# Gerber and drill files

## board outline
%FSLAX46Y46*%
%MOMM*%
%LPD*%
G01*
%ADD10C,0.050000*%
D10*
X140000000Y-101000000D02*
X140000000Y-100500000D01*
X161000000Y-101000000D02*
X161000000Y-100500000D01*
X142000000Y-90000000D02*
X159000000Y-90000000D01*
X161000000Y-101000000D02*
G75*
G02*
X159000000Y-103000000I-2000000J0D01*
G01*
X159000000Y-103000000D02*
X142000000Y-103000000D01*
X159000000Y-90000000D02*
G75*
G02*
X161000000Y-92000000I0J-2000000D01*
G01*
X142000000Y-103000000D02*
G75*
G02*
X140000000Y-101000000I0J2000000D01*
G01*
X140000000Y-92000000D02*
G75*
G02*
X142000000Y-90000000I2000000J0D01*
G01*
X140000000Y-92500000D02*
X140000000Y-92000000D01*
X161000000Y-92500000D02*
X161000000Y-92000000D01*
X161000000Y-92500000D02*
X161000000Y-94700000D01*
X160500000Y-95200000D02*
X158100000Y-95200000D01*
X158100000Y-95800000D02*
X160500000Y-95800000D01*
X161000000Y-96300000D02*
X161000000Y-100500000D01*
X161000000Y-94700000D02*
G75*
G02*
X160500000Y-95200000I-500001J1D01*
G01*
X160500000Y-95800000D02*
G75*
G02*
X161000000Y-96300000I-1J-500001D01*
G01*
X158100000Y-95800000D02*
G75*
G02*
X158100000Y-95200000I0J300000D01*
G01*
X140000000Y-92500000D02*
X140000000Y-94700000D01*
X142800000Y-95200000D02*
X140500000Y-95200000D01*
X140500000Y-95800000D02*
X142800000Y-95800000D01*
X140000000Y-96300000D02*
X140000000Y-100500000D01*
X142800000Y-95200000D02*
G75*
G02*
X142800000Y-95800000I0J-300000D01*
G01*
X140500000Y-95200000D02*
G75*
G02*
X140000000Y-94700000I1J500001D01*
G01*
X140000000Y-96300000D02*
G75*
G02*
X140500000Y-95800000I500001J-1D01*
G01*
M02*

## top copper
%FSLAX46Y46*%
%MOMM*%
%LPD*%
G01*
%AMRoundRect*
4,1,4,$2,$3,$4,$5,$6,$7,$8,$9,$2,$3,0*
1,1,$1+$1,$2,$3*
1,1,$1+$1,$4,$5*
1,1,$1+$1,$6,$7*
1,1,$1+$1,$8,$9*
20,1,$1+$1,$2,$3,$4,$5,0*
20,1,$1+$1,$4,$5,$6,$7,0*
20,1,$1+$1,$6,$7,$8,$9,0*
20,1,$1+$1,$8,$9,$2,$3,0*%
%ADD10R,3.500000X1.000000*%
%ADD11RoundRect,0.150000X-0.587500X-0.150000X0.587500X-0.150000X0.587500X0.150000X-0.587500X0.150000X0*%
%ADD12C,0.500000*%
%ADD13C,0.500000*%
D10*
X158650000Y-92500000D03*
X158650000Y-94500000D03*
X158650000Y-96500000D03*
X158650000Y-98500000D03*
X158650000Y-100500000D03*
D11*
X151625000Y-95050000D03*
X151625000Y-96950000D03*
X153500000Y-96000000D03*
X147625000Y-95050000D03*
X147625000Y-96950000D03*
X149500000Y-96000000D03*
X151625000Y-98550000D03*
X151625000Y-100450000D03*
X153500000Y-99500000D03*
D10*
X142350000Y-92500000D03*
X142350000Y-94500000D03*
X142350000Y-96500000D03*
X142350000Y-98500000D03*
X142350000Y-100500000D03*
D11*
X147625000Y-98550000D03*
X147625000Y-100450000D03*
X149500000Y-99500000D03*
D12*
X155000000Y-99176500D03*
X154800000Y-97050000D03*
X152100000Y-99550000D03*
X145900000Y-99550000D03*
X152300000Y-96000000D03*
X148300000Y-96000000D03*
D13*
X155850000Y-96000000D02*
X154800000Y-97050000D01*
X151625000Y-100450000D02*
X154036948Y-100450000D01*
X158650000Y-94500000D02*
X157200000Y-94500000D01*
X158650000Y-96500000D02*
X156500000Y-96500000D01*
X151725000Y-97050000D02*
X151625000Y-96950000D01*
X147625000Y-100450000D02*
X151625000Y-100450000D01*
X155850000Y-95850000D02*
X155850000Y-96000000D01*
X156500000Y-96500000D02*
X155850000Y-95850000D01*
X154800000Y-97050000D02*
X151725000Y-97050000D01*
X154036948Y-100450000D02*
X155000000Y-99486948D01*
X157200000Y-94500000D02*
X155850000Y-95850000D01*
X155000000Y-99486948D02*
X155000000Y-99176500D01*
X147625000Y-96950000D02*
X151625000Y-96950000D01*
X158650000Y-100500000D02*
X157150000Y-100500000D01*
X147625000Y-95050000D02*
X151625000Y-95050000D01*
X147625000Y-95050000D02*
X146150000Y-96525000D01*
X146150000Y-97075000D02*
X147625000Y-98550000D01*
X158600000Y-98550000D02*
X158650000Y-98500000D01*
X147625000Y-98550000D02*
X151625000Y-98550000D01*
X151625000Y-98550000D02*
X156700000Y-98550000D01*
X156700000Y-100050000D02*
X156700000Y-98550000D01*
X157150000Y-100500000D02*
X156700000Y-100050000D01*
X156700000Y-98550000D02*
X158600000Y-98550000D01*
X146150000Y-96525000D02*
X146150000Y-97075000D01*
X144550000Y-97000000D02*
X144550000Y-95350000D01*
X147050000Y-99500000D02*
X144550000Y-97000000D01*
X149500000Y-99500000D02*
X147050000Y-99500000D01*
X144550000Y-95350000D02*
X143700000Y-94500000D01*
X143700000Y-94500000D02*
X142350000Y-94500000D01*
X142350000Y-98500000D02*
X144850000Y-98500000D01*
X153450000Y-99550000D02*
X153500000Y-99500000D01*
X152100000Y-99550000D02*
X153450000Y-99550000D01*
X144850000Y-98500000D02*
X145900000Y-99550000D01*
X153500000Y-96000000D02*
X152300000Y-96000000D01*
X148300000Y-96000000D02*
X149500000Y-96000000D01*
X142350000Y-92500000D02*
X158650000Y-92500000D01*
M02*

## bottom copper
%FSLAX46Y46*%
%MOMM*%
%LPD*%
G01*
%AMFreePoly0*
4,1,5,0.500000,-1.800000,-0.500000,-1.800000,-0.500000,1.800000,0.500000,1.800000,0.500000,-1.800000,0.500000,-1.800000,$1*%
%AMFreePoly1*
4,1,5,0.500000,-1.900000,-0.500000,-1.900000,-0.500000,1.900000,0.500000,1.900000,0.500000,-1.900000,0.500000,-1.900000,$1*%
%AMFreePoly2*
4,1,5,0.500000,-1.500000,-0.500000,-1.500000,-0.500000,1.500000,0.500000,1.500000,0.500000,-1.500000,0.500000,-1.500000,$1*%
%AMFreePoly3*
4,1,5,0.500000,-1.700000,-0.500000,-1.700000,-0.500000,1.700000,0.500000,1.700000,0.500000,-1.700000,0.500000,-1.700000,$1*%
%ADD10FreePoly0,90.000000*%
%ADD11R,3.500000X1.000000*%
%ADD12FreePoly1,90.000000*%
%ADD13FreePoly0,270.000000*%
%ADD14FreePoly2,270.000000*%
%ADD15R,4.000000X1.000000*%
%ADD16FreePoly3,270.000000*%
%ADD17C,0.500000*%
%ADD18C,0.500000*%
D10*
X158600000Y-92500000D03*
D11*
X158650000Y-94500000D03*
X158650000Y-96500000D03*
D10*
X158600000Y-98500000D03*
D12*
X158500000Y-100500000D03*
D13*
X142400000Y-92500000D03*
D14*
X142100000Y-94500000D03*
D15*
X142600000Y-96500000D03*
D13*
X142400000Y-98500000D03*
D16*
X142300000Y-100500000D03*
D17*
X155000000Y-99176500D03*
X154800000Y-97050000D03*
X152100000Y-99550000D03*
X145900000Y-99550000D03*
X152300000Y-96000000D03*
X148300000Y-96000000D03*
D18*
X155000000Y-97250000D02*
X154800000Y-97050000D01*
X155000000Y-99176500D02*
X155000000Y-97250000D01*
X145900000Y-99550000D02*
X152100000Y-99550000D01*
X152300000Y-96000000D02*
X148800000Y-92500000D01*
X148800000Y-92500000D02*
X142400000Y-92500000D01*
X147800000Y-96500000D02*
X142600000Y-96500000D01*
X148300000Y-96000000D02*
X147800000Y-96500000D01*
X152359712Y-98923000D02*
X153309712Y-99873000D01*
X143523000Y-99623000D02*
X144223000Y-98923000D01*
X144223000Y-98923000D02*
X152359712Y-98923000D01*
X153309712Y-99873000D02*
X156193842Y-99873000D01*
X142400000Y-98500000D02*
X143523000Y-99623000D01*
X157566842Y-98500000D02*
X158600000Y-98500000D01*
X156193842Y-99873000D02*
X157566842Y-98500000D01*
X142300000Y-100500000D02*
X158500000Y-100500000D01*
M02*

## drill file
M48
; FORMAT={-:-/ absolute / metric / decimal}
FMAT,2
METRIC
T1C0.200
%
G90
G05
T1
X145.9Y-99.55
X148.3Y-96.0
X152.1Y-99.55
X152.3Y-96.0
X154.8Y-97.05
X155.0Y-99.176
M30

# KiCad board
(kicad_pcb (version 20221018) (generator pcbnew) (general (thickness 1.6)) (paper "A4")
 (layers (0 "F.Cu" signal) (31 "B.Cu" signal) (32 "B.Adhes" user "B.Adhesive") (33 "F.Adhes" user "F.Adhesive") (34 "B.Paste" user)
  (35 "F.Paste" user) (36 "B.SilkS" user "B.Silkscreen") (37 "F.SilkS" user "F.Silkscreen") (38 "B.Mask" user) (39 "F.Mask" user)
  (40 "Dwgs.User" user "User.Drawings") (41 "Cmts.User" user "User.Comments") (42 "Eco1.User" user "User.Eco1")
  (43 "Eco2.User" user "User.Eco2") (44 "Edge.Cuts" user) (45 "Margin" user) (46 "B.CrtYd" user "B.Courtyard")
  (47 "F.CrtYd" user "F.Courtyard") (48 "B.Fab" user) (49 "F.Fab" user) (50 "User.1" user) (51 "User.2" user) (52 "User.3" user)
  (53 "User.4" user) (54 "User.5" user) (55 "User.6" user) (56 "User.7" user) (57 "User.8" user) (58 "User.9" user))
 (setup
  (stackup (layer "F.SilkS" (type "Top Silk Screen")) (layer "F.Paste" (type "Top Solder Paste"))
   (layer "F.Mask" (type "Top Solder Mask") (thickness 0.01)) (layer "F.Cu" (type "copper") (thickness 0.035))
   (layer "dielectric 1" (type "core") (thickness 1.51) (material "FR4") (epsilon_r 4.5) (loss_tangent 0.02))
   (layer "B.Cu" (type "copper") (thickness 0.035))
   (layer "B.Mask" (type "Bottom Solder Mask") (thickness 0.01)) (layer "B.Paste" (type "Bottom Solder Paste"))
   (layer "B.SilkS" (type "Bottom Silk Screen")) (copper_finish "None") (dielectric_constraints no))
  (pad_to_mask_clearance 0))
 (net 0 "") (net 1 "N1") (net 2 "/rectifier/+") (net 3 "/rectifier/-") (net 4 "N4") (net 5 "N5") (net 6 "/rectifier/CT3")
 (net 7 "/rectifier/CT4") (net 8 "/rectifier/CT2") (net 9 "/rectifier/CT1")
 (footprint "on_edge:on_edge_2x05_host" (layer "F.Cu") (at 161 96.5 -90)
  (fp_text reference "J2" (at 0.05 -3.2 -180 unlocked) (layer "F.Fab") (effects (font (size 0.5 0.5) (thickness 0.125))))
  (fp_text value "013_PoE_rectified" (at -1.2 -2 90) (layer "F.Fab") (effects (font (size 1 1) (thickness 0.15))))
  (fp_line (start -4 0) (end -1.8 0) (stroke (width 0.05) (type solid)) (layer "Edge.Cuts"))
  (fp_line (start -1.3 0.5) (end -1.3 2.9) (stroke (width 0.05) (type solid)) (layer "Edge.Cuts"))
  (fp_line (start -0.7 2.9) (end -0.7 0.5) (stroke (width 0.05) (type solid)) (layer "Edge.Cuts"))
  (fp_line (start -0.2 0) (end 4 0) (stroke (width 0.05) (type solid)) (layer "Edge.Cuts"))
  (fp_arc (start -1.8 0) (mid -1.446447 0.146447) (end -1.3 0.5) (stroke (width 0.05) (type solid)) (layer "Edge.Cuts"))
  (fp_arc (start -0.7 0.5) (mid -0.553553 0.146447) (end -0.2 0) (stroke (width 0.05) (type solid)) (layer "Edge.Cuts"))
  (fp_arc (start -0.7 2.9) (mid -1 3.2) (end -1.3 2.9) (stroke (width 0.05) (type solid)) (layer "Edge.Cuts"))
  (pad "1" smd rect (at -4 2.35 270) (size 1 3.5) (layers "F.Cu" "F.Mask") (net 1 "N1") (zone_connect 0))
  (pad "2" smd rect (at -2 2.35 270) (size 1 3.5) (layers "F.Cu" "F.Mask") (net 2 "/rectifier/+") (zone_connect 0))
  (pad "3" smd rect (at 0 2.35 270) (size 1 3.5) (layers "F.Cu" "F.Mask") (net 2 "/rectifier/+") (zone_connect 0))
  (pad "4" smd rect (at 2 2.35 270) (size 1 3.5) (layers "F.Cu" "F.Mask") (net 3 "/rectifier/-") (zone_connect 0))
  (pad "5" smd rect (at 4 2.35 270) (size 1 3.5) (layers "F.Cu" "F.Mask") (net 3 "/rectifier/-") (zone_connect 0))
  (pad "6" smd custom (at -4 2.4 90) (size 1 3.6) (layers "B.Cu" "B.Mask") (zone_connect 0) (options (clearance outline) (anchor rect))
   (primitives))
  (pad "7" smd rect (at -2 2.35 90) (size 1 3.5) (layers "B.Cu" "B.Mask") (zone_connect 0))
  (pad "8" smd rect (at 0 2.35 90) (size 1 3.5) (layers "B.Cu" "B.Mask") (zone_connect 0))
  (pad "9" smd custom (at 2 2.4 90) (size 1 3.6) (layers "B.Cu" "B.Mask") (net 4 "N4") (zone_connect 0)
   (options (clearance outline) (anchor rect)) (primitives))
  (pad "10" smd custom (at 4 2.5 90) (size 1 3.8) (layers "B.Cu" "B.Mask") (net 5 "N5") (zone_connect 0)
   (options (clearance outline) (anchor rect)) (primitives))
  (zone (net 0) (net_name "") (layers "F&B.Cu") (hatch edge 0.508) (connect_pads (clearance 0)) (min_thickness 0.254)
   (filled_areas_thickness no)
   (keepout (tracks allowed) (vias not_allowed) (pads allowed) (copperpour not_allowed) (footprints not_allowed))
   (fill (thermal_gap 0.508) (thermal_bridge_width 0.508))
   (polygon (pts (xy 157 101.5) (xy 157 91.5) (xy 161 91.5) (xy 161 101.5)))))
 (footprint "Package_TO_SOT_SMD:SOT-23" (layer "F.Cu") (at 152.5625 96)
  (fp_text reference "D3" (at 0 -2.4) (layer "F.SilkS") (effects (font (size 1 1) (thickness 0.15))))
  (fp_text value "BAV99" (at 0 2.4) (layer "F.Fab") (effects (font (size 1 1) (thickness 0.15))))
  (pad "1" smd roundrect (at -0.9375 -0.95) (size 1.475 0.6) (layers "F.Cu" "F.Paste" "F.Mask") (roundrect_rratio 0.25)
   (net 3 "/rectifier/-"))
  (pad "2" smd roundrect (at -0.9375 0.95) (size 1.475 0.6) (layers "F.Cu" "F.Paste" "F.Mask") (roundrect_rratio 0.25)
   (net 2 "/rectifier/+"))
  (pad "3" smd roundrect (at 0.9375 0) (size 1.475 0.6) (layers "F.Cu" "F.Paste" "F.Mask") (roundrect_rratio 0.25) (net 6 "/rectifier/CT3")))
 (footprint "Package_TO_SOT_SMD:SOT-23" (layer "F.Cu") (at 148.5625 96)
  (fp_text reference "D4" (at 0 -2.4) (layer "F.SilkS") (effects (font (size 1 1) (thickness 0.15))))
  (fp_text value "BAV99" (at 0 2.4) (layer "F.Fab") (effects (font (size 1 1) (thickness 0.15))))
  (pad "1" smd roundrect (at -0.9375 -0.95) (size 1.475 0.6) (layers "F.Cu" "F.Paste" "F.Mask") (roundrect_rratio 0.25)
   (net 3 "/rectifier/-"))
  (pad "2" smd roundrect (at -0.9375 0.95) (size 1.475 0.6) (layers "F.Cu" "F.Paste" "F.Mask") (roundrect_rratio 0.25)
   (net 2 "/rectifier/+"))
  (pad "3" smd roundrect (at 0.9375 0) (size 1.475 0.6) (layers "F.Cu" "F.Paste" "F.Mask") (roundrect_rratio 0.25) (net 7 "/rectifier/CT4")))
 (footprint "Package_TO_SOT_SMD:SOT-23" (layer "F.Cu") (at 152.5625 99.5)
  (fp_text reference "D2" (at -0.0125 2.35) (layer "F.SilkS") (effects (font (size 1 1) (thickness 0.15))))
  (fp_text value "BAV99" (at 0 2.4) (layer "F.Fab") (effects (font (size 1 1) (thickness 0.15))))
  (pad "1" smd roundrect (at -0.9375 -0.95) (size 1.475 0.6) (layers "F.Cu" "F.Paste" "F.Mask") (roundrect_rratio 0.25)
   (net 3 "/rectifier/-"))
  (pad "2" smd roundrect (at -0.9375 0.95) (size 1.475 0.6) (layers "F.Cu" "F.Paste" "F.Mask") (roundrect_rratio 0.25)
   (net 2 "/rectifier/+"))
  (pad "3" smd roundrect (at 0.9375 0) (size 1.475 0.6) (layers "F.Cu" "F.Paste" "F.Mask") (roundrect_rratio 0.25) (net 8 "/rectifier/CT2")))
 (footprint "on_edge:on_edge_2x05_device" (layer "F.Cu") (at 140 96.5 -90)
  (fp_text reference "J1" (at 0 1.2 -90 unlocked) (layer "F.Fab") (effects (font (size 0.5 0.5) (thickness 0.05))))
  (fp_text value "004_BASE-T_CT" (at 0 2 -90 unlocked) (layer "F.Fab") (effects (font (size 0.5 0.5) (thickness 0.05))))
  (fp_line (start -4 0) (end -1.8 0) (stroke (width 0.05) (type solid)) (layer "Edge.Cuts"))
  (fp_line (start -1.3 -2.8) (end -1.3 -0.5) (stroke (width 0.05) (type solid)) (layer "Edge.Cuts"))
  (fp_line (start -0.7 -0.5) (end -0.7 -2.8) (stroke (width 0.05) (type solid)) (layer "Edge.Cuts"))
  (fp_line (start -0.2 0) (end 4 0) (stroke (width 0.05) (type solid)) (layer "Edge.Cuts"))
  (fp_arc (start -1.3 -2.8) (mid -1 -3.1) (end -0.7 -2.8) (stroke (width 0.05) (type solid)) (layer "Edge.Cuts"))
  (fp_arc (start -1.3 -0.5) (mid -1.446447 -0.146447) (end -1.8 0) (stroke (width 0.05) (type solid)) (layer "Edge.Cuts"))
  (fp_arc (start -0.2 0) (mid -0.553553 -0.146447) (end -0.7 -0.5) (stroke (width 0.05) (type solid)) (layer "Edge.Cuts"))
  (pad "1" smd rect (at -4 -2.35 90) (size 1 3.5) (layers "F.Cu" "F.Mask") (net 1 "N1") (zone_connect 0))
  (pad "2" smd rect (at -2 -2.35 270) (size 1 3.5) (layers "F.Cu" "F.Mask") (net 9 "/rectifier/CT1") (zone_connect 0))
  (pad "3" smd rect (at 0 -2.35 270) (size 1 3.5) (layers "F.Cu" "F.Mask") (zone_connect 0))
  (pad "4" smd rect (at 2 -2.35 90) (size 1 3.5) (layers "F.Cu" "F.Mask") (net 8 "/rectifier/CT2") (zone_connect 0))
  (pad "5" smd rect (at 4 -2.35 90) (size 1 3.5) (layers "F.Cu" "F.Mask") (zone_connect 0))
  (pad "6" smd custom (at -4 -2.4 270) (size 1 3.6) (layers "B.Cu" "B.Mask") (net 6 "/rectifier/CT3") (zone_connect 0)
   (options (clearance outline) (anchor rect)) (primitives))
  (pad "7" smd custom (at -2 -2.1 270) (size 1 3) (layers "B.Cu" "B.Mask") (zone_connect 0) (options (clearance outline) (anchor rect))
   (primitives))
  (pad "8" smd rect (at 0 -2.6 270) (size 1 4) (layers "B.Cu" "B.Mask") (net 7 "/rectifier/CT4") (zone_connect 0))
  (pad "9" smd custom (at 2 -2.4 270) (size 1 3.6) (layers "B.Cu" "B.Mask") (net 4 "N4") (zone_connect 0)
   (options (clearance outline) (anchor rect)) (primitives))
  (pad "10" smd custom (at 4 -2.3 270) (size 1 3.4) (layers "B.Cu" "B.Mask") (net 5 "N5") (zone_connect 0)
   (options (clearance outline) (anchor rect)) (primitives))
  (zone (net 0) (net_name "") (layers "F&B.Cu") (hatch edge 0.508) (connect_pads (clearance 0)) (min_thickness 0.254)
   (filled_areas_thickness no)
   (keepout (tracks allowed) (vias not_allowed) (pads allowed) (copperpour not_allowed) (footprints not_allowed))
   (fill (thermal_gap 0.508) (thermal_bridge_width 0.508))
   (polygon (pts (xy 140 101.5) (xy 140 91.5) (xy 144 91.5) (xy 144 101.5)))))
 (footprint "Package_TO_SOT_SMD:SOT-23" (layer "F.Cu") (at 148.5625 99.5)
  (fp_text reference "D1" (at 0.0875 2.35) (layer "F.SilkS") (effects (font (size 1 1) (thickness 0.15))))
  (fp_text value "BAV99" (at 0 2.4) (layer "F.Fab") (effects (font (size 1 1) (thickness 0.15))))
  (pad "1" smd roundrect (at -0.9375 -0.95) (size 1.475 0.6) (layers "F.Cu" "F.Paste" "F.Mask") (roundrect_rratio 0.25)
   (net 3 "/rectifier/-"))
  (pad "2" smd roundrect (at -0.9375 0.95) (size 1.475 0.6) (layers "F.Cu" "F.Paste" "F.Mask") (roundrect_rratio 0.25)
   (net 2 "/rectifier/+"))
  (pad "3" smd roundrect (at 0.9375 0) (size 1.475 0.6) (layers "F.Cu" "F.Paste" "F.Mask") (roundrect_rratio 0.25) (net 9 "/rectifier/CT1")))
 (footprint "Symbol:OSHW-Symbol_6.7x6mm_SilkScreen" (layer "B.Cu") (at 152.45 99.75 180)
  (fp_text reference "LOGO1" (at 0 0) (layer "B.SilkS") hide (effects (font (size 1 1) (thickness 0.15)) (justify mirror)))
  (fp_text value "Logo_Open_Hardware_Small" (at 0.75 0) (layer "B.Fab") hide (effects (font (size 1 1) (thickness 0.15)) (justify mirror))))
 (gr_line (start 140 101) (end 140 100.5) (stroke (width 0.05) (type solid)) (layer "Edge.Cuts"))
 (gr_line (start 161 101) (end 161 100.5) (stroke (width 0.05) (type solid)) (layer "Edge.Cuts"))
 (gr_line (start 142 90) (end 159 90) (stroke (width 0.05) (type solid)) (layer "Edge.Cuts"))
 (gr_arc (start 161 101) (mid 160.414214 102.414214) (end 159 103) (stroke (width 0.05) (type solid)) (layer "Edge.Cuts"))
 (gr_line (start 159 103) (end 142 103) (stroke (width 0.05) (type solid)) (layer "Edge.Cuts"))
 (gr_arc (start 159 90) (mid 160.414214 90.585786) (end 161 92) (stroke (width 0.05) (type solid)) (layer "Edge.Cuts"))
 (gr_arc (start 142 103) (mid 140.585786 102.414214) (end 140 101) (stroke (width 0.05) (type solid)) (layer "Edge.Cuts"))
 (gr_arc (start 140 92) (mid 140.585786 90.585786) (end 142 90) (stroke (width 0.05) (type solid)) (layer "Edge.Cuts"))
 (gr_line (start 140 92.5) (end 140 92) (stroke (width 0.05) (type solid)) (layer "Edge.Cuts"))
 (gr_line (start 161 92.5) (end 161 92) (stroke (width 0.05) (type solid)) (layer "Edge.Cuts"))
 (segment (start 155.85 96) (end 154.8 97.05) (width 0.5) (layer "F.Cu") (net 2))
 (segment (start 151.625 100.45) (end 154.036948 100.45) (width 0.5) (layer "F.Cu") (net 2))
 (segment (start 158.65 94.5) (end 157.2 94.5) (width 0.5) (layer "F.Cu") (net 2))
 (segment (start 158.65 96.5) (end 156.5 96.5) (width 0.5) (layer "F.Cu") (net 2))
 (segment (start 151.725 97.05) (end 151.625 96.95) (width 0.5) (layer "F.Cu") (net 2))
 (segment (start 147.625 100.45) (end 151.625 100.45) (width 0.5) (layer "F.Cu") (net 2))
 (segment (start 155.85 95.85) (end 155.85 96) (width 0.5) (layer "F.Cu") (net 2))
 (segment (start 156.5 96.5) (end 155.85 95.85) (width 0.5) (layer "F.Cu") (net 2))
 (segment (start 154.8 97.05) (end 151.725 97.05) (width 0.5) (layer "F.Cu") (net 2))
 (segment (start 154.036948 100.45) (end 155 99.486948) (width 0.5) (layer "F.Cu") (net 2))
 (segment (start 157.2 94.5) (end 155.85 95.85) (width 0.5) (layer "F.Cu") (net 2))
 (segment (start 155 99.486948) (end 155 99.1765) (width 0.5) (layer "F.Cu") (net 2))
 (segment (start 147.625 96.95) (end 151.625 96.95) (width 0.5) (layer "F.Cu") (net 2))
 (via (at 155 99.1765) (size 0.5) (drill 0.2) (layers "F.Cu" "B.Cu") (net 2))
 (via (at 154.8 97.05) (size 0.5) (drill 0.2) (layers "F.Cu" "B.Cu") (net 2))
 (segment (start 155 97.25) (end 154.8 97.05) (width 0.5) (layer "B.Cu") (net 2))
 (segment (start 155 99.1765) (end 155 97.25) (width 0.5) (layer "B.Cu") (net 2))
 (segment (start 158.65 100.5) (end 157.15 100.5) (width 0.5) (layer "F.Cu") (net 3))
 (segment (start 147.625 95.05) (end 151.625 95.05) (width 0.5) (layer "F.Cu") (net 3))
 (segment (start 147.625 95.05) (end 146.15 96.525) (width 0.5) (layer "F.Cu") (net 3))
 (segment (start 146.15 97.075) (end 147.625 98.55) (width 0.5) (layer "F.Cu") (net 3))
 (segment (start 158.6 98.55) (end 158.65 98.5) (width 0.5) (layer "F.Cu") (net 3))
 (segment (start 147.625 98.55) (end 151.625 98.55) (width 0.5) (layer "F.Cu") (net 3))
 (segment (start 151.625 98.55) (end 156.7 98.55) (width 0.5) (layer "F.Cu") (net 3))
 (segment (start 156.7 100.05) (end 156.7 98.55) (width 0.5) (layer "F.Cu") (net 3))
 (segment (start 157.15 100.5) (end 156.7 100.05) (width 0.5) (layer "F.Cu") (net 3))
 (segment (start 156.7 98.55) (end 158.6 98.55) (width 0.5) (layer "F.Cu") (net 3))
 (segment (start 146.15 96.525) (end 146.15 97.075) (width 0.5) (layer "F.Cu") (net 3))
 (segment (start 144.55 97) (end 144.55 95.35) (width 0.5) (layer "F.Cu") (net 9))
 (segment (start 147.05 99.5) (end 144.55 97) (width 0.5) (layer "F.Cu") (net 9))
 (segment (start 149.5 99.5) (end 147.05 99.5) (width 0.5) (layer "F.Cu") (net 9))
 (segment (start 144.55 95.35) (end 143.7 94.5) (width 0.5) (layer "F.Cu") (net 9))
 (segment (start 143.7 94.5) (end 142.35 94.5) (width 0.5) (layer "F.Cu") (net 9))
 (segment (start 142.35 98.5) (end 144.85 98.5) (width 0.5) (layer "F.Cu") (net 8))
 (segment (start 153.45 99.55) (end 153.5 99.5) (width 0.5) (layer "F.Cu") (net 8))
 (segment (start 152.1 99.55) (end 153.45 99.55) (width 0.5) (layer "F.Cu") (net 8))
 (segment (start 144.85 98.5) (end 145.9 99.55) (width 0.5) (layer "F.Cu") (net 8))
 (via (at 152.1 99.55) (size 0.5) (drill 0.2) (layers "F.Cu" "B.Cu") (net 8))
 (via (at 145.9 99.55) (size 0.5) (drill 0.2) (layers "F.Cu" "B.Cu") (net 8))
 (segment (start 145.9 99.55) (end 152.1 99.55) (width 0.5) (layer "B.Cu") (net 8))
 (segment (start 153.5 96) (end 152.3 96) (width 0.5) (layer "F.Cu") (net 6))
 (via (at 152.3 96) (size 0.5) (drill 0.2) (layers "F.Cu" "B.Cu") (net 6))
 (segment (start 152.3 96) (end 148.8 92.5) (width 0.5) (layer "B.Cu") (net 6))
 (segment (start 148.8 92.5) (end 142.4 92.5) (width 0.5) (layer "B.Cu") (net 6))
 (segment (start 148.3 96) (end 149.5 96) (width 0.5) (layer "F.Cu") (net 7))
 (via (at 148.3 96) (size 0.5) (drill 0.2) (layers "F.Cu" "B.Cu") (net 7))
 (segment (start 147.8 96.5) (end 142.6 96.5) (width 0.5) (layer "B.Cu") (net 7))
 (segment (start 148.3 96) (end 147.8 96.5) (width 0.5) (layer "B.Cu") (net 7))
 (segment (start 142.35 92.5) (end 158.65 92.5) (width 0.5) (layer "F.Cu") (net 1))
 (segment (start 152.359712 98.923) (end 153.309712 99.873) (width 0.5) (layer "B.Cu") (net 4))
 (segment (start 143.523 99.623) (end 144.223 98.923) (width 0.5) (layer "B.Cu") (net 4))
 (segment (start 144.223 98.923) (end 152.359712 98.923) (width 0.5) (layer "B.Cu") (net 4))
 (segment (start 153.309712 99.873) (end 156.193842 99.873) (width 0.5) (layer "B.Cu") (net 4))
 (segment (start 142.4 98.5) (end 143.523 99.623) (width 0.5) (layer "B.Cu") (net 4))
 (segment (start 157.566842 98.5) (end 158.6 98.5) (width 0.5) (layer "B.Cu") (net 4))
 (segment (start 156.193842 99.873) (end 157.566842 98.5) (width 0.5) (layer "B.Cu") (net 4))
 (segment (start 142.3 100.5) (end 158.5 100.5) (width 0.5) (layer "B.Cu") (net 5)))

